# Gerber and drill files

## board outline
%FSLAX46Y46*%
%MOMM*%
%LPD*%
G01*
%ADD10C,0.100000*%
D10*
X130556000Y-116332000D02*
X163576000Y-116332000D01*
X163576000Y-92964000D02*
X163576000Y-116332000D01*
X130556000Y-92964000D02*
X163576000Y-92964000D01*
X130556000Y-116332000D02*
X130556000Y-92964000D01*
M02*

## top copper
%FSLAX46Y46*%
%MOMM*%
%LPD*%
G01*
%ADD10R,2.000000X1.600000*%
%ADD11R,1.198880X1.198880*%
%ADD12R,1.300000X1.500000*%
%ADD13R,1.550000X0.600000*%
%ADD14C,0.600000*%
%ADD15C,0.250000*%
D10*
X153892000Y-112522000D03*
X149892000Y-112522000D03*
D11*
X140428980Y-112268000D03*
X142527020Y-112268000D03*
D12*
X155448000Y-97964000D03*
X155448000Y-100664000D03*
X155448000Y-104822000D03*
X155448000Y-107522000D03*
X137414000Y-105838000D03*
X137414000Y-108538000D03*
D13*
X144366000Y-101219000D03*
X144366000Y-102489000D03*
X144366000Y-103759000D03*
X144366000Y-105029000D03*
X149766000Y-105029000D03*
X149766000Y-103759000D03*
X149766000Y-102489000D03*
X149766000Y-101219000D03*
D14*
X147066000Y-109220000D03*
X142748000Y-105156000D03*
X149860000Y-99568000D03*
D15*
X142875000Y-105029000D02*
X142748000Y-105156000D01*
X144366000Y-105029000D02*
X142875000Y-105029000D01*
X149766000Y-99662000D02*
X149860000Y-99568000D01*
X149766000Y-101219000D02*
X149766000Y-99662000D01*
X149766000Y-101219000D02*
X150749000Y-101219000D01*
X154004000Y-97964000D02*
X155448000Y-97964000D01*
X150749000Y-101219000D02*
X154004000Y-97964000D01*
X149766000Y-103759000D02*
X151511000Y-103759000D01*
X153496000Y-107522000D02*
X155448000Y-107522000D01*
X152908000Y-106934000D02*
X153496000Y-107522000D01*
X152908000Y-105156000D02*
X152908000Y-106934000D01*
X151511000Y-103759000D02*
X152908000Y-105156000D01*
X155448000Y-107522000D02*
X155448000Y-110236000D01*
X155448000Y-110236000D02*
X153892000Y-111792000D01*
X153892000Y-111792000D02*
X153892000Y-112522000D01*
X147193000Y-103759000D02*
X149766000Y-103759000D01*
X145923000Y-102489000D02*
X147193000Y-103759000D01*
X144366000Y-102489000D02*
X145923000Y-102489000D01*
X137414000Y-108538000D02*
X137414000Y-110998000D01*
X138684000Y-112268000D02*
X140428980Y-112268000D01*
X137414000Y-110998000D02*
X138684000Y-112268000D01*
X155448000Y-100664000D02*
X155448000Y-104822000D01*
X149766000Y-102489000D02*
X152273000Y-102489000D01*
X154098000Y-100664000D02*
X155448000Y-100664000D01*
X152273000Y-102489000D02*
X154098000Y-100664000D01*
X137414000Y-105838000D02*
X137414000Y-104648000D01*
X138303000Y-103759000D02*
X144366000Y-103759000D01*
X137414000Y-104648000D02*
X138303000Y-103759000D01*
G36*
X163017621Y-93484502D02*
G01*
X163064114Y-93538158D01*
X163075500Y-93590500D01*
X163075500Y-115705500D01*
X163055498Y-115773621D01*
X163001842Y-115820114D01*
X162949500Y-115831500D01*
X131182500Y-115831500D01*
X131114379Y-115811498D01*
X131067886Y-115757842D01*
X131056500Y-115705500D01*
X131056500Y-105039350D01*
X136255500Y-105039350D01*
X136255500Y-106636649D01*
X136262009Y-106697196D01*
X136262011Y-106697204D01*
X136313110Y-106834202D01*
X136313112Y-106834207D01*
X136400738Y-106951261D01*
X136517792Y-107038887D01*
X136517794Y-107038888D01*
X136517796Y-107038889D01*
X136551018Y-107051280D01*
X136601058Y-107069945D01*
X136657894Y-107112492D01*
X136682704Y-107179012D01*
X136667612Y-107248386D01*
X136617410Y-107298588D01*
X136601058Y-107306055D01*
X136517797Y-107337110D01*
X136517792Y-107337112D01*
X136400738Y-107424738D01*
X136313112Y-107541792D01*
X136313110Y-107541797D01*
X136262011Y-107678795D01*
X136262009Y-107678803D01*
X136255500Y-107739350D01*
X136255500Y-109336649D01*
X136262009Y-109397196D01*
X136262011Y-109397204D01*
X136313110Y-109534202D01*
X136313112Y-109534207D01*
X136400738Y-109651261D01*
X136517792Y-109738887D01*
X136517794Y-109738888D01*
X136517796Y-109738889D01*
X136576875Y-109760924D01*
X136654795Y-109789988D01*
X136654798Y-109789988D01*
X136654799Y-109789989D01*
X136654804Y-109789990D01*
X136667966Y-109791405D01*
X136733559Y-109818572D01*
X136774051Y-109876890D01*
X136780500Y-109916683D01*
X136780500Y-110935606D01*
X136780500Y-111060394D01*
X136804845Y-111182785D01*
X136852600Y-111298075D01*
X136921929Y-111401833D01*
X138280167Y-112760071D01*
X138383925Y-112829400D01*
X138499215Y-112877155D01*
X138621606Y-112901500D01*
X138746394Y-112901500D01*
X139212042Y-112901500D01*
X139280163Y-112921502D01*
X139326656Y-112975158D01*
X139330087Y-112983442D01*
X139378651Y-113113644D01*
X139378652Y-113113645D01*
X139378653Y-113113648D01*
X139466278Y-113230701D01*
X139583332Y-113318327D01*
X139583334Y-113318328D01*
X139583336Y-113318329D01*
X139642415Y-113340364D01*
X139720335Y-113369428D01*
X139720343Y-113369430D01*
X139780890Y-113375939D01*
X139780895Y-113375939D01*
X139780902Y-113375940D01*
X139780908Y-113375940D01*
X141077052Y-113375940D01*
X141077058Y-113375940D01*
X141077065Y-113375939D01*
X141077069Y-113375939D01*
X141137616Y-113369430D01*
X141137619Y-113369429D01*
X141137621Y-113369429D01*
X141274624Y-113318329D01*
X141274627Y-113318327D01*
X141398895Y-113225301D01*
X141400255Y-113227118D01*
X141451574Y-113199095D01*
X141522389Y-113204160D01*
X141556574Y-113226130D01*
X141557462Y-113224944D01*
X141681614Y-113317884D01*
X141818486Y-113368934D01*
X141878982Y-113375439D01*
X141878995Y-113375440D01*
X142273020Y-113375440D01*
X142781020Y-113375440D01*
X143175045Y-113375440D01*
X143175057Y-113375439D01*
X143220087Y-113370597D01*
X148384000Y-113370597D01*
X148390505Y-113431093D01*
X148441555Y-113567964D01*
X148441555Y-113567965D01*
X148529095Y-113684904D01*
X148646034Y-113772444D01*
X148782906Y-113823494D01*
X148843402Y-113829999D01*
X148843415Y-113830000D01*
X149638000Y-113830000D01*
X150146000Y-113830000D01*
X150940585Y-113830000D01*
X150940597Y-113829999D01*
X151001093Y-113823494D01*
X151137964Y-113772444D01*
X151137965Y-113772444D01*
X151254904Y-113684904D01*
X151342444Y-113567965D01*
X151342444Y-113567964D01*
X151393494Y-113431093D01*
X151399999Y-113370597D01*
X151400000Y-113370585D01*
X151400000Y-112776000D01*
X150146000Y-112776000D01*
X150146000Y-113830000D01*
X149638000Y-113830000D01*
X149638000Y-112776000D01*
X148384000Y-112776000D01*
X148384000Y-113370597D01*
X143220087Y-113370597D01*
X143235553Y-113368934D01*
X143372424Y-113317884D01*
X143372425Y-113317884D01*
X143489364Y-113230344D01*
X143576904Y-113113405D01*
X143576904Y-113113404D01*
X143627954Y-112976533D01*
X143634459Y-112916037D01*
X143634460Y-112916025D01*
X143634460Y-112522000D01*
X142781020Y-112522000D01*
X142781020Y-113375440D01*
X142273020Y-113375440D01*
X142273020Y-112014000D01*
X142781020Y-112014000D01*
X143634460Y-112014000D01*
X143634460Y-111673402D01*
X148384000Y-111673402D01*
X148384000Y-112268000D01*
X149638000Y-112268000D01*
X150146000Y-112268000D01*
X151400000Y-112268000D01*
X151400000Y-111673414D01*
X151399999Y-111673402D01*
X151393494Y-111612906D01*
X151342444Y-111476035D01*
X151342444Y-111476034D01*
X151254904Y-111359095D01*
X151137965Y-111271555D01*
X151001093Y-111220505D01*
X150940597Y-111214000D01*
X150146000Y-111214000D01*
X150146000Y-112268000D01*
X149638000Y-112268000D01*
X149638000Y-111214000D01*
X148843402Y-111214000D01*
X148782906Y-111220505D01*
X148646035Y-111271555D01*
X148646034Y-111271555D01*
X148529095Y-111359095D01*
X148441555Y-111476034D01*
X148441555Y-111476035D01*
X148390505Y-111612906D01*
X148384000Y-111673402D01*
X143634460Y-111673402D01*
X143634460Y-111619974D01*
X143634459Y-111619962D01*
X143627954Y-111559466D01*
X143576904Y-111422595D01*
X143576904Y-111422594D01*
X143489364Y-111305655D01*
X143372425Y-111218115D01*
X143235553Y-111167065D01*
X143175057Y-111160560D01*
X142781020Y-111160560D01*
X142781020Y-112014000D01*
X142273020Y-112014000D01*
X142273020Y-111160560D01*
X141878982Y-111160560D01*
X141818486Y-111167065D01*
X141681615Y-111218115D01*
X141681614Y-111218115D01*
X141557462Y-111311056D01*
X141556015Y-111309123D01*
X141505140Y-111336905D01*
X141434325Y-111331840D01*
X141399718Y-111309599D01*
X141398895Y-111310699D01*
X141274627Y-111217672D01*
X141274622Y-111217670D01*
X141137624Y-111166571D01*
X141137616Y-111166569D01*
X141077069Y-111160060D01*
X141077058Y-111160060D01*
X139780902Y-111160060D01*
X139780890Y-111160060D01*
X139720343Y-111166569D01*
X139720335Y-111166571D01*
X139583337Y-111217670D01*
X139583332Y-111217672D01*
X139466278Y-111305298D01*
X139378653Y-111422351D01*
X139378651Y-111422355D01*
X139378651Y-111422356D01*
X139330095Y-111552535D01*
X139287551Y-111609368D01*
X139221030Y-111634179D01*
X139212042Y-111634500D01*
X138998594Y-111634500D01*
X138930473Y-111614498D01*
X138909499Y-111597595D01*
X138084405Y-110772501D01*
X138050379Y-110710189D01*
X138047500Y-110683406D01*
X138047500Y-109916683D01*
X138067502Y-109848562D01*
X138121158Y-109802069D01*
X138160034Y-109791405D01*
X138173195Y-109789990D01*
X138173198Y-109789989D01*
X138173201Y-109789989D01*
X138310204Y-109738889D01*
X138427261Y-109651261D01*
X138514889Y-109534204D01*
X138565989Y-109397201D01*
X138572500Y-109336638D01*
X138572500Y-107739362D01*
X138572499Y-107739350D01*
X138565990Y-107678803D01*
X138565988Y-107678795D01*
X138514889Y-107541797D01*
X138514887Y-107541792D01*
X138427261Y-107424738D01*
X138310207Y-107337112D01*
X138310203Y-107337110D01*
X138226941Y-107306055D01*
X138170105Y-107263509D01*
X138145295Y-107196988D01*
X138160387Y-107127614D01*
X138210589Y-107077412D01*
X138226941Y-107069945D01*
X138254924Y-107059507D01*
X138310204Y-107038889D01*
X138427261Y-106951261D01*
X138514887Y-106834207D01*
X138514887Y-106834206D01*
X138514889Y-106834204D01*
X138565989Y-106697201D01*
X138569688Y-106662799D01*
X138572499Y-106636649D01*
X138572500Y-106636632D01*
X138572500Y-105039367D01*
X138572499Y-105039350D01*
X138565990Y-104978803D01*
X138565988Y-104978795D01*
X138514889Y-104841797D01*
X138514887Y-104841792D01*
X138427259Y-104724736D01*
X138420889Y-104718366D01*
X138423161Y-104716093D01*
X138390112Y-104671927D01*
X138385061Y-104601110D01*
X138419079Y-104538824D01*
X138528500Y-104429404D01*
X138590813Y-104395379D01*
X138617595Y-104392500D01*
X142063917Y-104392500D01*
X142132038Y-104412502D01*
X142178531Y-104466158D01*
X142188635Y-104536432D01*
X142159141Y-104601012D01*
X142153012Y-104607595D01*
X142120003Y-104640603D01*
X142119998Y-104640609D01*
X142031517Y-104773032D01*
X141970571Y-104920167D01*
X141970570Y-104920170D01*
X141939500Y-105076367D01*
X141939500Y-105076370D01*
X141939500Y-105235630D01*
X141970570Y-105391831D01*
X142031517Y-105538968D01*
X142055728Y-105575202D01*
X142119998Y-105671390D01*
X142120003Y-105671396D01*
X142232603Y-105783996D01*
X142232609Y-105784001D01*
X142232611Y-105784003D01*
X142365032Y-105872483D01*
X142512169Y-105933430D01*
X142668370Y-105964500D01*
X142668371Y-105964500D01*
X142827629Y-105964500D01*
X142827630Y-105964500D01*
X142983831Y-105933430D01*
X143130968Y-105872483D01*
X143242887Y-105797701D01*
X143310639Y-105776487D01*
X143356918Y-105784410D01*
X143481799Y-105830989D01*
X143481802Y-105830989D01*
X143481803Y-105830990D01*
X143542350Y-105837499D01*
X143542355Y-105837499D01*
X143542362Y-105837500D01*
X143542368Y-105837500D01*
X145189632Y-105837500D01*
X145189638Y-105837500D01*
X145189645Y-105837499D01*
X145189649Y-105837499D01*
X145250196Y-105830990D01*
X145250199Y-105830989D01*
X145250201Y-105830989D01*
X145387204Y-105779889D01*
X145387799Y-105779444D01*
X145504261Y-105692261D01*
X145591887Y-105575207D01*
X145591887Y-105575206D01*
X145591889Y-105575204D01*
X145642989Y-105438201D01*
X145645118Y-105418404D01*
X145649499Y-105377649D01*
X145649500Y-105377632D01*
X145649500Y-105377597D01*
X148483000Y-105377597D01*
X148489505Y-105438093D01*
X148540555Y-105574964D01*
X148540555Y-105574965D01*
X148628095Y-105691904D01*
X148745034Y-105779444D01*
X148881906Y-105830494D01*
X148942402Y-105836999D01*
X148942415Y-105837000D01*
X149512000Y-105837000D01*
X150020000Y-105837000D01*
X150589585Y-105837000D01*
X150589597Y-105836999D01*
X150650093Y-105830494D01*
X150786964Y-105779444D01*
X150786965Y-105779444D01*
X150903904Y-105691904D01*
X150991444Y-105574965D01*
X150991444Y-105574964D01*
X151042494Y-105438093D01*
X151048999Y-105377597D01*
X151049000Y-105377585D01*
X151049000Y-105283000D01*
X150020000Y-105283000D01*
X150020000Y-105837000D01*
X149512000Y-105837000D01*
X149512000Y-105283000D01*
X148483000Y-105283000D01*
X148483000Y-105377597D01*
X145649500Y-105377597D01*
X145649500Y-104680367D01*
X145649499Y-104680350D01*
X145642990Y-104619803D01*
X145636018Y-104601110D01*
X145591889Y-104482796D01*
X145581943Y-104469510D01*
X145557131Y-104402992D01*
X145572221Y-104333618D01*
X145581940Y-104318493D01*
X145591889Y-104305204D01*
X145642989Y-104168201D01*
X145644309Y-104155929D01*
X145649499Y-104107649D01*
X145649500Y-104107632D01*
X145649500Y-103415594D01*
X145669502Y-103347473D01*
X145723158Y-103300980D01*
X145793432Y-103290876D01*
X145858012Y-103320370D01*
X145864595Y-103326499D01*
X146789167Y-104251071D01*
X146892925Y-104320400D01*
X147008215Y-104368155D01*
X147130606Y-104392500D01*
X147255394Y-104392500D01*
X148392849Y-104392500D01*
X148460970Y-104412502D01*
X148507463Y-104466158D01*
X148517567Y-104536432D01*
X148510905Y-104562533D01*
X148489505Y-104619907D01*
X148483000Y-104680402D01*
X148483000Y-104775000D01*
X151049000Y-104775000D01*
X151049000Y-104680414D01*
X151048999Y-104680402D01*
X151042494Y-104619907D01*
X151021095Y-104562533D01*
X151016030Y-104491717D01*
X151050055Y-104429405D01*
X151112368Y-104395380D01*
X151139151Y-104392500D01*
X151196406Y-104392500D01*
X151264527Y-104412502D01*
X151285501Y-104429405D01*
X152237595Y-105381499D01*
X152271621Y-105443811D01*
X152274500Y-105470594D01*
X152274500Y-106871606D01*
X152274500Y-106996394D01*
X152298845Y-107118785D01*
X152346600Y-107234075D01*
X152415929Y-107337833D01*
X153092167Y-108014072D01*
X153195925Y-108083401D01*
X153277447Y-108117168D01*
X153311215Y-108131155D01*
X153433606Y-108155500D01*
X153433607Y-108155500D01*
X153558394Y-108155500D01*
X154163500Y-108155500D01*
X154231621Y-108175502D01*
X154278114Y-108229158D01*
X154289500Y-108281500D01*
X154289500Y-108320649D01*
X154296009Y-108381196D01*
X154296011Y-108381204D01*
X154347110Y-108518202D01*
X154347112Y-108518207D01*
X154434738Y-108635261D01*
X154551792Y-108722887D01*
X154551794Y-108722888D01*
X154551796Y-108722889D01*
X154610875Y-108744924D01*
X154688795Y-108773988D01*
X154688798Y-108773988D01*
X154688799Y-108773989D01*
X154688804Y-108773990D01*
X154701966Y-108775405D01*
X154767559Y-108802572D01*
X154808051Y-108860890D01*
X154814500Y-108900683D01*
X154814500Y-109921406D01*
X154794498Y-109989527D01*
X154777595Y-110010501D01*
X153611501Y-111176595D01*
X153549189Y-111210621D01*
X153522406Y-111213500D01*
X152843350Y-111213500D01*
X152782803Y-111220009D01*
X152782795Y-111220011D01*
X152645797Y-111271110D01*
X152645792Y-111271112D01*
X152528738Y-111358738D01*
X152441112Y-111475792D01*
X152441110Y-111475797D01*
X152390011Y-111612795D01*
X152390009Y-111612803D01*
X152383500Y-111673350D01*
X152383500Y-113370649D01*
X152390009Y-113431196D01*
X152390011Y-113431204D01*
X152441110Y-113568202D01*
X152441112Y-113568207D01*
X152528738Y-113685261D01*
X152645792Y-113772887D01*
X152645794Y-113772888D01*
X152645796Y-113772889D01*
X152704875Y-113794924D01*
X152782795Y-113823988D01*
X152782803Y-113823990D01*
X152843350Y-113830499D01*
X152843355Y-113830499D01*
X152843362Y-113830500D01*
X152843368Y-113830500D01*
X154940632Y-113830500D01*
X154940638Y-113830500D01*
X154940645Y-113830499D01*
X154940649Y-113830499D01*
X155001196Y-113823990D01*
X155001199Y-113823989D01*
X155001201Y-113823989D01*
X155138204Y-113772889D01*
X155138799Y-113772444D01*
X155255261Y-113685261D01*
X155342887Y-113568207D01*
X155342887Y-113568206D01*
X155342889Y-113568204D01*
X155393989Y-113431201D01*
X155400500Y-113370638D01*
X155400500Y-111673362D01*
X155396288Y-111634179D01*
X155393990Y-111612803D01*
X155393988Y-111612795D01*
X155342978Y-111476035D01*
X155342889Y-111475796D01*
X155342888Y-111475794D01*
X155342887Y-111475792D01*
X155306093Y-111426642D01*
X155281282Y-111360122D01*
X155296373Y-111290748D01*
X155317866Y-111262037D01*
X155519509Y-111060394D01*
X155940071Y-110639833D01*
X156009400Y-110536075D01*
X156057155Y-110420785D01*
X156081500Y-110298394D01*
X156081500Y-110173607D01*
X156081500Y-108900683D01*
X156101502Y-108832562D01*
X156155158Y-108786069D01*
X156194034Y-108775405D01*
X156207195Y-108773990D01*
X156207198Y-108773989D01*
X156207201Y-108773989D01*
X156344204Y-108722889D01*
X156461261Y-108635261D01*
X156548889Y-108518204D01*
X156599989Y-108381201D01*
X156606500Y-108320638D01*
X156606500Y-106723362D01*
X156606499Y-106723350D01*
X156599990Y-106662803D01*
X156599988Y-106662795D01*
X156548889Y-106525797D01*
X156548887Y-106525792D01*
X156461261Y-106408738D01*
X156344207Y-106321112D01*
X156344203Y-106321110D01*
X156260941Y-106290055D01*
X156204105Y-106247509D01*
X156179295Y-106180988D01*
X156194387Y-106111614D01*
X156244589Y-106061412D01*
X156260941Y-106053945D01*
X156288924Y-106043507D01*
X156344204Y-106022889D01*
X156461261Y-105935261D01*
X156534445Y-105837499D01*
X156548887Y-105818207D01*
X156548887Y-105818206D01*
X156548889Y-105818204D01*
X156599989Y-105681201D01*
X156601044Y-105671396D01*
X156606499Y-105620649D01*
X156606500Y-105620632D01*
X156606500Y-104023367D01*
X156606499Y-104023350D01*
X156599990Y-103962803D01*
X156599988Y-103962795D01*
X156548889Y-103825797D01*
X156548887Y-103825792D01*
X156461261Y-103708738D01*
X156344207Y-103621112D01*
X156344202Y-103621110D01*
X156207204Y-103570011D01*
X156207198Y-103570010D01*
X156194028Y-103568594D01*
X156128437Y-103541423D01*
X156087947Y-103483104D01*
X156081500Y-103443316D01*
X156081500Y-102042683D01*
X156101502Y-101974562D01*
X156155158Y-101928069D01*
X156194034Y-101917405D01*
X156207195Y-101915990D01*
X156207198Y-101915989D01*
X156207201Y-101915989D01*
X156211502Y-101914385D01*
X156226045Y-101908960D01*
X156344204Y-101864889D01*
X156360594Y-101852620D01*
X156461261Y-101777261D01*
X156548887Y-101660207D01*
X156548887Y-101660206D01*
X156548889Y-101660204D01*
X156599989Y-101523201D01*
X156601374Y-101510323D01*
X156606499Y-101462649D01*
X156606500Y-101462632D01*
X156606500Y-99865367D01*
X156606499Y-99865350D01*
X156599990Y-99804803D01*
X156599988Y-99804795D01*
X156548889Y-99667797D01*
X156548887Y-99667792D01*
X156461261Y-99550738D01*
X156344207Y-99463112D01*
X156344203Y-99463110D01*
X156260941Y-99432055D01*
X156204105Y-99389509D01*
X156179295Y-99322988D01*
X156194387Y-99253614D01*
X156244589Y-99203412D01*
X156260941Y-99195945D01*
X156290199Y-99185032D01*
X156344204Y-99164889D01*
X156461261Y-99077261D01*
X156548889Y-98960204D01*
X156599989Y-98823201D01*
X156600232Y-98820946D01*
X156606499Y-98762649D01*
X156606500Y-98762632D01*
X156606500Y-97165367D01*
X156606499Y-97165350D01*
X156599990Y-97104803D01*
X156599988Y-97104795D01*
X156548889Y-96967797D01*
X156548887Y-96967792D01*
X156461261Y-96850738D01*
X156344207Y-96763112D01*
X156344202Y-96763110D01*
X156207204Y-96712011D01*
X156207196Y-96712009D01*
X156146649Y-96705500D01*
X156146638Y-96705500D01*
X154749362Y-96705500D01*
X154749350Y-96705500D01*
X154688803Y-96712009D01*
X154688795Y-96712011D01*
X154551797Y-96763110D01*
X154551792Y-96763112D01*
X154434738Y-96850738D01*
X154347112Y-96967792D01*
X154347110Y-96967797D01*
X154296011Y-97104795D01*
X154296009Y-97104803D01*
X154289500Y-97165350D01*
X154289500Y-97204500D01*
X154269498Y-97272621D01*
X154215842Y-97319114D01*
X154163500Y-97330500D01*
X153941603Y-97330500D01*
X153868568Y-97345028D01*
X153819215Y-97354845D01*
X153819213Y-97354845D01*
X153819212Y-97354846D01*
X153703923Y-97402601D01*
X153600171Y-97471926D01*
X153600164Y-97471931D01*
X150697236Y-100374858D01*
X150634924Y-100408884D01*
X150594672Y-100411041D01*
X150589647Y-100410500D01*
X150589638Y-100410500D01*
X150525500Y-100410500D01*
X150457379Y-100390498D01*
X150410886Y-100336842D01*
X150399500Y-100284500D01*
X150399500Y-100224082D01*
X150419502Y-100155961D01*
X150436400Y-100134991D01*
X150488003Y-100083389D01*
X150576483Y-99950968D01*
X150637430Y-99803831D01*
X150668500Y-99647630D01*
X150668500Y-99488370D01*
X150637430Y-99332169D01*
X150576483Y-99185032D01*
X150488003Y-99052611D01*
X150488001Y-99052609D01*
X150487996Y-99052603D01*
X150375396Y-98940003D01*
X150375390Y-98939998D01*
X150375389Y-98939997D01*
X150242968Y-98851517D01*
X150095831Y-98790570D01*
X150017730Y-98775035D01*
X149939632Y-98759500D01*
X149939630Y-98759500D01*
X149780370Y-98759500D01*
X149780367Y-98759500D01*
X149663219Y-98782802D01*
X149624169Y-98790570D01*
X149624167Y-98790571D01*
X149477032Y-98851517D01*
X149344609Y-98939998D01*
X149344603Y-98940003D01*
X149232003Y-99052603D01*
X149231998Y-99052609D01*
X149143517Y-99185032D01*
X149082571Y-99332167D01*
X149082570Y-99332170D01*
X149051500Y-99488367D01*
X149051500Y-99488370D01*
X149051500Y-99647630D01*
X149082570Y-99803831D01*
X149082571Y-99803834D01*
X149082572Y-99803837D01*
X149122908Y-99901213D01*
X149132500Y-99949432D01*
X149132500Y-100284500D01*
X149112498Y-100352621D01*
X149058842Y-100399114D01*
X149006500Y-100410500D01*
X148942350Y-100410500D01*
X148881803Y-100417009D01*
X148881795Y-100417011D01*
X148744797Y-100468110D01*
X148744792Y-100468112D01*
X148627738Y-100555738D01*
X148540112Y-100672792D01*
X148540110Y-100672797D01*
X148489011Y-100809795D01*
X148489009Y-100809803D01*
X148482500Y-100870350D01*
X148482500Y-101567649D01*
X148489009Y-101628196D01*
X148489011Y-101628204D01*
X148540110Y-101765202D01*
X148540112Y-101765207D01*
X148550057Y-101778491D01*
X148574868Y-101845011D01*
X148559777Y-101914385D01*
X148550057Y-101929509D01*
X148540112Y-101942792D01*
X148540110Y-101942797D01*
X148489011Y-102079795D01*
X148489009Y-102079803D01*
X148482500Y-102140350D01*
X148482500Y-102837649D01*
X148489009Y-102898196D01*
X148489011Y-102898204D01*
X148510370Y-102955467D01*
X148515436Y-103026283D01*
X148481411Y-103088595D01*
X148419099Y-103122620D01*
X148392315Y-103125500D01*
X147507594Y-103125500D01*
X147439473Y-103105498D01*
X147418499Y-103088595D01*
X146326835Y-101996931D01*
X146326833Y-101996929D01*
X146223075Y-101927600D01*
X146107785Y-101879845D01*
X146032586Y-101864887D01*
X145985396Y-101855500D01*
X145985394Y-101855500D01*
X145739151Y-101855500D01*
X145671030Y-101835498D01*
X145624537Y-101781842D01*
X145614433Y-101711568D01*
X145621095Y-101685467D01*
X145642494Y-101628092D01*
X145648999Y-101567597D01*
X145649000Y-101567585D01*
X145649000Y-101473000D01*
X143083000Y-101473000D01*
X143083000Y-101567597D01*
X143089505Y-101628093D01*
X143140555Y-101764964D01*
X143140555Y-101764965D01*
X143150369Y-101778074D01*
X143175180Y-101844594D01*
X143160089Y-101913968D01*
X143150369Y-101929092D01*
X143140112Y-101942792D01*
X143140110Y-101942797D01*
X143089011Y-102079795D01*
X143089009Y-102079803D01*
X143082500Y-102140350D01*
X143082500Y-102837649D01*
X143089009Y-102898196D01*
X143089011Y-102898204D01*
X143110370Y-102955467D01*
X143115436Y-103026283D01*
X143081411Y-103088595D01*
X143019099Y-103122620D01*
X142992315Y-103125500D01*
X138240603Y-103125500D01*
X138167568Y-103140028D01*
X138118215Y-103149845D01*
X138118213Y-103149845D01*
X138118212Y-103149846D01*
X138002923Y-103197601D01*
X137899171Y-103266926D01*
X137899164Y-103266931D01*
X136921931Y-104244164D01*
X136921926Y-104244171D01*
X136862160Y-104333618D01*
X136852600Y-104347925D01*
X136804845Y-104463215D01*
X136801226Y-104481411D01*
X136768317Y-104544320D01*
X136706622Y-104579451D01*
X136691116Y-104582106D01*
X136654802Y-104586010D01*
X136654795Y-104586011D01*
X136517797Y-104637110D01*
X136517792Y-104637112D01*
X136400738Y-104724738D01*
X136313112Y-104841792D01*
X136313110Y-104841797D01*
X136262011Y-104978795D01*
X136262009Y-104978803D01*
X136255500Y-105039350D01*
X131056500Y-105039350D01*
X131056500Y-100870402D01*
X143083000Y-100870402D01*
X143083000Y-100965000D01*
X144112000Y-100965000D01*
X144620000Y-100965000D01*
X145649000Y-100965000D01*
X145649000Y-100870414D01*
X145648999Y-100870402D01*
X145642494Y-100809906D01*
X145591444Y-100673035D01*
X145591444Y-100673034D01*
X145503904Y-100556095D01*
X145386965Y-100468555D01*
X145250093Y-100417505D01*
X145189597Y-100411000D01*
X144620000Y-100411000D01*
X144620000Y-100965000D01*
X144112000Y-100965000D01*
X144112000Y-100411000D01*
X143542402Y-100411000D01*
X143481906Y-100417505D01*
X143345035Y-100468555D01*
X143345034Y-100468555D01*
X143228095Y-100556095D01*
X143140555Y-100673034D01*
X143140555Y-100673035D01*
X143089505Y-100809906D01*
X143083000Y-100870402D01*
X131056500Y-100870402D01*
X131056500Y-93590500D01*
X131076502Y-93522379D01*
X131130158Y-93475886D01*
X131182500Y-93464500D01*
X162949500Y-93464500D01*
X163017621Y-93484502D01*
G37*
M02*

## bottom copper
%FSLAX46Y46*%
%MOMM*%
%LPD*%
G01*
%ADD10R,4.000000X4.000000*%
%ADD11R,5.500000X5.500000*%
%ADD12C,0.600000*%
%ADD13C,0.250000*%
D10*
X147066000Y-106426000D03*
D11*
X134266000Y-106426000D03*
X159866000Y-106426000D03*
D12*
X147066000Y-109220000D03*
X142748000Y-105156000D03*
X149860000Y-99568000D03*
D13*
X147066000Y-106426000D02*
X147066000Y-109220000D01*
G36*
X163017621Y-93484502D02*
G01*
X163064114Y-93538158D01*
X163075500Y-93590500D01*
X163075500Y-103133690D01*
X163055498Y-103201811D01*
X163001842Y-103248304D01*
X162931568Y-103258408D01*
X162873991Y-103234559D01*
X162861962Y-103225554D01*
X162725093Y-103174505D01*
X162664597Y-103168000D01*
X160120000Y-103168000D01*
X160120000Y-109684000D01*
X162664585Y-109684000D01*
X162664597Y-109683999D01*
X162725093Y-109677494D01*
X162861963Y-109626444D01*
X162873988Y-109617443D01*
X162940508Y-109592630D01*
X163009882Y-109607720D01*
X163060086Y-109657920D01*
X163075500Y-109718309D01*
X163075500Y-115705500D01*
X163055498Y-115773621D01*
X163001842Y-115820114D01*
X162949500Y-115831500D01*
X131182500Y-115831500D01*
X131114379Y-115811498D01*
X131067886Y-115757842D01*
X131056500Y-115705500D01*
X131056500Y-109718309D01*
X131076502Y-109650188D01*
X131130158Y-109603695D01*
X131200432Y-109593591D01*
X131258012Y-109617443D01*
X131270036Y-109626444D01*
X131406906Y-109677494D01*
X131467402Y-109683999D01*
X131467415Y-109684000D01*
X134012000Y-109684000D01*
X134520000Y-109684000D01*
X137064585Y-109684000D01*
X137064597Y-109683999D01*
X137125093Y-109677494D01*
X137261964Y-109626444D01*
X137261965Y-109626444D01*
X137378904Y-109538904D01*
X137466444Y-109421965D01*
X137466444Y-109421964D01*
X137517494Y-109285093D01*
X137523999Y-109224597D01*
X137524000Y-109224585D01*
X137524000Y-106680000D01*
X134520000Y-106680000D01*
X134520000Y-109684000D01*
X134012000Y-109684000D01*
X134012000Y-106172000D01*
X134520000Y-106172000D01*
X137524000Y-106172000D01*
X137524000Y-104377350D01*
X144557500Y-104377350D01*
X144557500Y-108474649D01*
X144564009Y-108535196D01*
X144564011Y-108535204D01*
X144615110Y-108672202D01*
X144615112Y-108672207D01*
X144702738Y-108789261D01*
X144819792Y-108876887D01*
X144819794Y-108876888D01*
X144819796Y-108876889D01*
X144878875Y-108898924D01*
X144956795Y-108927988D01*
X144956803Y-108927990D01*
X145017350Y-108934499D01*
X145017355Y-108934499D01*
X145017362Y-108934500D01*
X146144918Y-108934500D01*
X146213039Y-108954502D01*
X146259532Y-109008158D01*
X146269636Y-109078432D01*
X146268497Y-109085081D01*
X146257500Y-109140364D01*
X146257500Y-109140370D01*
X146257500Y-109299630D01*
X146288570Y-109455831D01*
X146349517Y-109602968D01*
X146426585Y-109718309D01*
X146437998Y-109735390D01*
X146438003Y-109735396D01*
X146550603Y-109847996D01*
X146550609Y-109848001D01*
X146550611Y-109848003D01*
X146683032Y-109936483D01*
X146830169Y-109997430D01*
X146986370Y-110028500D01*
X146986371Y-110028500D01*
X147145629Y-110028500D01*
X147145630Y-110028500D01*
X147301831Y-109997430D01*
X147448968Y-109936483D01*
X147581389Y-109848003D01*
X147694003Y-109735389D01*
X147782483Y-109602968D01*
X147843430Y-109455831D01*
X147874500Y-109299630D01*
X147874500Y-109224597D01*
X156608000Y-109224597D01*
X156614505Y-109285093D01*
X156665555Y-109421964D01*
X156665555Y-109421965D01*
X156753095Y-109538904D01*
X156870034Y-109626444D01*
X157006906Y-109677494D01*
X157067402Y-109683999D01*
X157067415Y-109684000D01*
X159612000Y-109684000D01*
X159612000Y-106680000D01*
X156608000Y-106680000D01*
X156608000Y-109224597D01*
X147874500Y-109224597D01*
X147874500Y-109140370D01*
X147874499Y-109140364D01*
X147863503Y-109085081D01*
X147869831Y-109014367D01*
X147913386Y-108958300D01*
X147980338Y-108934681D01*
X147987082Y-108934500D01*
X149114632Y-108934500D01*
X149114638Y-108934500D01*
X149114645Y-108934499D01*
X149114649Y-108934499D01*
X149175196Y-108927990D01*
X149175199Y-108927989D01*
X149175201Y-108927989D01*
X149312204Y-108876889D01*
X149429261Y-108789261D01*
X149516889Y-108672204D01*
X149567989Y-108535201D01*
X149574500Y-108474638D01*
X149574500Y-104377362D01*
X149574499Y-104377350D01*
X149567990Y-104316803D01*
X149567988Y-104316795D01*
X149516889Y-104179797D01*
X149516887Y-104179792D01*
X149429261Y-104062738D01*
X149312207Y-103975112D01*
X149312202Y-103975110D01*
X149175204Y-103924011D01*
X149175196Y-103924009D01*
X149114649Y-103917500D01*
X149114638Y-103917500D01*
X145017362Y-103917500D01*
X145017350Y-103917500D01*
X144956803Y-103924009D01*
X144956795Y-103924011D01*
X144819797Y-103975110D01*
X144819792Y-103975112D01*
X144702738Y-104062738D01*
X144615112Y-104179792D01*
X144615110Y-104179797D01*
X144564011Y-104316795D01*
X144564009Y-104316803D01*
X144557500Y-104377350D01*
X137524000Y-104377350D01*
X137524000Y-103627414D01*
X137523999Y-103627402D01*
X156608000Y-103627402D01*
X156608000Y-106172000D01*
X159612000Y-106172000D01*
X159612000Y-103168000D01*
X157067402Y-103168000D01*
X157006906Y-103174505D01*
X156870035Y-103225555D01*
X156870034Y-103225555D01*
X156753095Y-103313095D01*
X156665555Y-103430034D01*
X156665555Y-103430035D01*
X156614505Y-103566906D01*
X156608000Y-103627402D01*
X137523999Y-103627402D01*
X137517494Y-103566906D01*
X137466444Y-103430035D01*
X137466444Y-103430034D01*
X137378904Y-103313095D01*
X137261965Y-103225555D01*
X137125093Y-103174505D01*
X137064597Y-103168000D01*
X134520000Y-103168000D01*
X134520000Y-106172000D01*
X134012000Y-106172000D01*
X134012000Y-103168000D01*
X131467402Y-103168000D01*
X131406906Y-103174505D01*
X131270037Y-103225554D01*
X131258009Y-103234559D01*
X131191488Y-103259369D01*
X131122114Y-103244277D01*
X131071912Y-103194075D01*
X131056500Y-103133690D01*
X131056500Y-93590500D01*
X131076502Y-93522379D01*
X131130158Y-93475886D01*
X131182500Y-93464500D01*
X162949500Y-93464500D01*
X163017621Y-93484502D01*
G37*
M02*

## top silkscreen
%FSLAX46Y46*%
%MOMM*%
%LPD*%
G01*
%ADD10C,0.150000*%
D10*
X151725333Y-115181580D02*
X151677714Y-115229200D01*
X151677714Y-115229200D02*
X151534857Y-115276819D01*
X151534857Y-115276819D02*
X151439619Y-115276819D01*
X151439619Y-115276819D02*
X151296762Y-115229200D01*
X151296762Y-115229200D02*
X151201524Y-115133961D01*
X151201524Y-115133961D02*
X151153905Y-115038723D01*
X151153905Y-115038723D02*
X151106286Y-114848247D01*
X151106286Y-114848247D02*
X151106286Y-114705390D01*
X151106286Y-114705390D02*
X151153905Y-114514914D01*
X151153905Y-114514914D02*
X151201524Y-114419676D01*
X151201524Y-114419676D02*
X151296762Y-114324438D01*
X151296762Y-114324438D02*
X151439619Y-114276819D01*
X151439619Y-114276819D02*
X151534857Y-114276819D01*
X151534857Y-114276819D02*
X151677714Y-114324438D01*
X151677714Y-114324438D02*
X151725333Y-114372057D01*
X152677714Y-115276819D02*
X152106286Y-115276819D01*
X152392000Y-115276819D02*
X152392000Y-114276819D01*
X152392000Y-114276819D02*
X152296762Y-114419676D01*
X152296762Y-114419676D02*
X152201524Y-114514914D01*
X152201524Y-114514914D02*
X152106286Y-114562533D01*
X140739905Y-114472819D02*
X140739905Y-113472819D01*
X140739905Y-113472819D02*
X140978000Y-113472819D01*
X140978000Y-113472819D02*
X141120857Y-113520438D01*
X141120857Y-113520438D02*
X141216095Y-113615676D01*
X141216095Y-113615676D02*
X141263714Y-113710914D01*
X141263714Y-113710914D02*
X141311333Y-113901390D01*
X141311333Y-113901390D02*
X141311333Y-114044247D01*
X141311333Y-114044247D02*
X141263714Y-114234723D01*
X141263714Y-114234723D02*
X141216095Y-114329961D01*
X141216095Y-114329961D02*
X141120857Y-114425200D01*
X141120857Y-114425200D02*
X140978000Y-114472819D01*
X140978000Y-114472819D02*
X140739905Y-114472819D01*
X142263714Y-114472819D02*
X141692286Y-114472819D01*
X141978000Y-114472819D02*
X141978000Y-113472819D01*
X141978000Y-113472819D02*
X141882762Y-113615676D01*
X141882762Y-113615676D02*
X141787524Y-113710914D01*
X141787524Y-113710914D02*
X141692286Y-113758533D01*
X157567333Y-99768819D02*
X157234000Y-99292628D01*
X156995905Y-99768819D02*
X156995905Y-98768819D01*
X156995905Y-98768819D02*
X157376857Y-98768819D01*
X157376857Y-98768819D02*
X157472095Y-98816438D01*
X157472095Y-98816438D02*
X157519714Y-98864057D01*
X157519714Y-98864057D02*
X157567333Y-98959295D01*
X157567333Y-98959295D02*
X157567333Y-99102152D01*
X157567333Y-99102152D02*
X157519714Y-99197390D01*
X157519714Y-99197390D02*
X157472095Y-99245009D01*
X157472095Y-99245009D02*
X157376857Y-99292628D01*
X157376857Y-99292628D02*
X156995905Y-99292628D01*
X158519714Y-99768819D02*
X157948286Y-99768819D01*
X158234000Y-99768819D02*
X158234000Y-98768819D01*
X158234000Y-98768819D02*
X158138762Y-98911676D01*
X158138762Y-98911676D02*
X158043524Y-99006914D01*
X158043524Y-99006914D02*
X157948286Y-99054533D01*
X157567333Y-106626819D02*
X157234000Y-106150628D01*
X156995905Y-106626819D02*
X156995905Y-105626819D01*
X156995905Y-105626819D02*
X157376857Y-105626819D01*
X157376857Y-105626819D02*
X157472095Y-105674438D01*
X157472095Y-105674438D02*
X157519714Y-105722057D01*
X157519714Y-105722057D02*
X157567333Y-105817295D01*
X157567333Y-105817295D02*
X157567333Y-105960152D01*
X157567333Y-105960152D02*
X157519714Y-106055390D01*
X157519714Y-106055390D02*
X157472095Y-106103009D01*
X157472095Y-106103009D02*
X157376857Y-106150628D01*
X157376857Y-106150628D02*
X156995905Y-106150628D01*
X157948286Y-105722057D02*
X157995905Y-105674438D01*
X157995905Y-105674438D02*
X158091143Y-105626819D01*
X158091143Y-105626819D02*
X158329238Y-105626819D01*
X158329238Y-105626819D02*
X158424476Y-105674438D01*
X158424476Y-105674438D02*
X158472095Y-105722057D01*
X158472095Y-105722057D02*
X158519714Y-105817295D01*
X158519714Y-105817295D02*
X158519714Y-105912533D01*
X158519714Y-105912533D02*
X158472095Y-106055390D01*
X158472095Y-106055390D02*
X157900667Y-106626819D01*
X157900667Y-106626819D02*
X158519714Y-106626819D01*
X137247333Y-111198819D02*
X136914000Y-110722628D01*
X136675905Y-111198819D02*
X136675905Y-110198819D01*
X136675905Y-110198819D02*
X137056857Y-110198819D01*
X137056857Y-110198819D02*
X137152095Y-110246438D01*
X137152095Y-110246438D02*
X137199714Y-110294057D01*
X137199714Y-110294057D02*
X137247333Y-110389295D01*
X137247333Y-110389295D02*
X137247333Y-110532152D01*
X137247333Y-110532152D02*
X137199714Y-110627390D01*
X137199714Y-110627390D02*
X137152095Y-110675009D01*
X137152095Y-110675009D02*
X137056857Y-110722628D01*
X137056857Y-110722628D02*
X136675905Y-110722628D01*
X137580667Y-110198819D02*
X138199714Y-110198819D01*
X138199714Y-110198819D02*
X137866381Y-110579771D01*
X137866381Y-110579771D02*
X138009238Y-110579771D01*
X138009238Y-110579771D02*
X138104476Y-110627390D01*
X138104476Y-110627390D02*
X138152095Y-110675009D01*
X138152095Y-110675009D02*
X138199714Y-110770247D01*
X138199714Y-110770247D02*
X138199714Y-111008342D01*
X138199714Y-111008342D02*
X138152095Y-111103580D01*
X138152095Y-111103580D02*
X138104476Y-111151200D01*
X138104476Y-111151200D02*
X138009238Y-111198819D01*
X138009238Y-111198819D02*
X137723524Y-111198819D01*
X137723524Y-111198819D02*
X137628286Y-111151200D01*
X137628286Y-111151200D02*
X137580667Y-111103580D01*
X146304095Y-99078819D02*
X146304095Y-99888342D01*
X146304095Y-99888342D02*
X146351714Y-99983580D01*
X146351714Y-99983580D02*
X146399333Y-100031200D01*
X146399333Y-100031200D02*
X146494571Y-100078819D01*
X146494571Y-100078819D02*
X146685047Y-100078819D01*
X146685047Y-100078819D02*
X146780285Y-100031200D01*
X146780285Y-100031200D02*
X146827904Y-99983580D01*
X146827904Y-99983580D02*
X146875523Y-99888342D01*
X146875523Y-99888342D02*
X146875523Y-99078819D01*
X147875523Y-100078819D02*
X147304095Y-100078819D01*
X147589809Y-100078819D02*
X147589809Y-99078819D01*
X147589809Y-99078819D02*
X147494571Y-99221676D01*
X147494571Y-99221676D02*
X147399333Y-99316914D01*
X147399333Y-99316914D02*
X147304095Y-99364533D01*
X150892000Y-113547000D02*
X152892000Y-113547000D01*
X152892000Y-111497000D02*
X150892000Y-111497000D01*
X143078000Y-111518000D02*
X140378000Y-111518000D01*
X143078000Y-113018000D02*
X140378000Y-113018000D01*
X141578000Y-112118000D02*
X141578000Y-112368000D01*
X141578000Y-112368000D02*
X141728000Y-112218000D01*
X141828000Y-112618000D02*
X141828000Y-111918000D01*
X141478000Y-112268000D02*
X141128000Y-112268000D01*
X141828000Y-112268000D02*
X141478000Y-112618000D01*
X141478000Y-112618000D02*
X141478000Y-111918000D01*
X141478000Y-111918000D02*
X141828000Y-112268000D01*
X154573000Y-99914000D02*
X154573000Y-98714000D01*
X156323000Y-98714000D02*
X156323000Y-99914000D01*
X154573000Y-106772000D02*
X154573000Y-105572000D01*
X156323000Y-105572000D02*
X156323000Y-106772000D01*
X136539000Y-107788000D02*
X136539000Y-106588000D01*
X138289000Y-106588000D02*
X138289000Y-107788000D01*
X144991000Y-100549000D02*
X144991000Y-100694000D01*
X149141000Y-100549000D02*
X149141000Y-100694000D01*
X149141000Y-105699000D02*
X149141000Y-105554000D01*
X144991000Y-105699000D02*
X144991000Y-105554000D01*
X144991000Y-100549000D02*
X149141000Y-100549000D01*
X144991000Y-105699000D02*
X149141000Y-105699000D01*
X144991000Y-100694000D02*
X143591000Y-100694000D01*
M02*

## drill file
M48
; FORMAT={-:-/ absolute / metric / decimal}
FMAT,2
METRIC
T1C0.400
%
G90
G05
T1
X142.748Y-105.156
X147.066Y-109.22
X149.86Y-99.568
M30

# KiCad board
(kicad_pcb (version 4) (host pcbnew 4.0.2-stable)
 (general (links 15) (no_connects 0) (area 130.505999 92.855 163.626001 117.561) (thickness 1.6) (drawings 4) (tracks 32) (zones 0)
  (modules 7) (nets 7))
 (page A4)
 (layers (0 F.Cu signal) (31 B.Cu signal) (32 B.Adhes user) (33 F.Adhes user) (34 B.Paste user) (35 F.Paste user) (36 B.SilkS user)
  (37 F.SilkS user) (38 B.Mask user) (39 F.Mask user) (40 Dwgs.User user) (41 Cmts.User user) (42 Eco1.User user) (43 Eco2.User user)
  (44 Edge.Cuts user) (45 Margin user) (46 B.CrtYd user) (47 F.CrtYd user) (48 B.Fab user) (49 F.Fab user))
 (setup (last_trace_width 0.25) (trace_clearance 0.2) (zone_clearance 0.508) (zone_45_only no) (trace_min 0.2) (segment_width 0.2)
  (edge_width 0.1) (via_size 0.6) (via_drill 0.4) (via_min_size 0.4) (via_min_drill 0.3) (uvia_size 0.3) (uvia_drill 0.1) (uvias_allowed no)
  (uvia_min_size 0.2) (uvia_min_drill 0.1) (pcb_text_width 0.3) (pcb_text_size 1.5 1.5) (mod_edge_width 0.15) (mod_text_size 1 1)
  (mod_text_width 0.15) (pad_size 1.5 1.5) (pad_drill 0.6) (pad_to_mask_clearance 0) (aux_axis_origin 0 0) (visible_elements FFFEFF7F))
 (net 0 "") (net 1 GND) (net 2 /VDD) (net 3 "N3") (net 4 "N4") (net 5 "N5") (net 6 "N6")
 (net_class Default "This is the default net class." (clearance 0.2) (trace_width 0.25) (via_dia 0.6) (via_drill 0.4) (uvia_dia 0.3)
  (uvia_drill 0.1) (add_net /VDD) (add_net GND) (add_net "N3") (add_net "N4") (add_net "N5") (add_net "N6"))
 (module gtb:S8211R (layer B.Cu) (at 147.066 106.426)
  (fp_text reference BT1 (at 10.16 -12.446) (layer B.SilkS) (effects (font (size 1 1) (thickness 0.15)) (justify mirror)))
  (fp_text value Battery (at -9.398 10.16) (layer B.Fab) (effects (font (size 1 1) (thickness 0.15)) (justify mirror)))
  (pad 2 smd rect (at 0 0) (size 4 4) (layers B.Cu B.Paste B.Mask) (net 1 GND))
  (pad 1 smd rect (at -12.8 0) (size 5.5 5.5) (layers B.Cu B.Paste B.Mask) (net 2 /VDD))
  (pad 1 smd rect (at 12.8 0) (size 5.5 5.5) (layers B.Cu B.Paste B.Mask) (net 2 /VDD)))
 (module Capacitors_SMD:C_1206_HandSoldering (layer F.Cu) (at 151.892 112.522 180)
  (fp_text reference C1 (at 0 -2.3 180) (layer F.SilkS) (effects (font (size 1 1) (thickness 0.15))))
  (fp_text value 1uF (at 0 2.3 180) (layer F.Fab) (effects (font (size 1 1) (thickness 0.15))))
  (fp_line (start 1 -1.025) (end -1 -1.025) (layer F.SilkS) (width 0.15))
  (fp_line (start -1 1.025) (end 1 1.025) (layer F.SilkS) (width 0.15))
  (pad 1 smd rect (at -2 0 180) (size 2 1.6) (layers F.Cu F.Paste F.Mask) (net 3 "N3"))
  (pad 2 smd rect (at 2 0 180) (size 2 1.6) (layers F.Cu F.Paste F.Mask) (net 1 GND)))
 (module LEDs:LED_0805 (layer F.Cu) (at 141.478 112.268 180)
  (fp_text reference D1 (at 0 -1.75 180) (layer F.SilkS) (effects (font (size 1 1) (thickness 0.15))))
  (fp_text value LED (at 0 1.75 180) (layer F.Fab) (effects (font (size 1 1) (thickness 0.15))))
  (fp_line (start -1.6 0.75) (end 1.1 0.75) (layer F.SilkS) (width 0.15))
  (fp_line (start -1.6 -0.75) (end 1.1 -0.75) (layer F.SilkS) (width 0.15))
  (fp_line (start -0.1 0.15) (end -0.1 -0.1) (layer F.SilkS) (width 0.15))
  (fp_line (start -0.1 -0.1) (end -0.25 0.05) (layer F.SilkS) (width 0.15))
  (fp_line (start -0.35 -0.35) (end -0.35 0.35) (layer F.SilkS) (width 0.15))
  (fp_line (start 0 0) (end 0.35 0) (layer F.SilkS) (width 0.15))
  (fp_line (start -0.35 0) (end 0 -0.35) (layer F.SilkS) (width 0.15))
  (fp_line (start 0 -0.35) (end 0 0.35) (layer F.SilkS) (width 0.15))
  (fp_line (start 0 0.35) (end -0.35 0) (layer F.SilkS) (width 0.15))
  (pad 2 smd rect (at 1.04902 0) (size 1.19888 1.19888) (layers F.Cu F.Paste F.Mask) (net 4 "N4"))
  (pad 1 smd rect (at -1.04902 0) (size 1.19888 1.19888) (layers F.Cu F.Paste F.Mask) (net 1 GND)))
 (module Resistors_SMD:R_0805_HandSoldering (layer F.Cu) (at 155.448 99.314 270)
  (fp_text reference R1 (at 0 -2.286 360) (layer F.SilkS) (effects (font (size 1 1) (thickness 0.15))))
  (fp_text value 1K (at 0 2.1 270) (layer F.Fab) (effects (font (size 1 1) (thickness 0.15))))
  (fp_line (start 0.6 0.875) (end -0.6 0.875) (layer F.SilkS) (width 0.15))
  (fp_line (start -0.6 -0.875) (end 0.6 -0.875) (layer F.SilkS) (width 0.15))
  (pad 1 smd rect (at -1.35 0 270) (size 1.5 1.3) (layers F.Cu F.Paste F.Mask) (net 2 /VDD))
  (pad 2 smd rect (at 1.35 0 270) (size 1.5 1.3) (layers F.Cu F.Paste F.Mask) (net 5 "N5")))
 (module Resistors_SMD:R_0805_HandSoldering (layer F.Cu) (at 155.448 106.172 270)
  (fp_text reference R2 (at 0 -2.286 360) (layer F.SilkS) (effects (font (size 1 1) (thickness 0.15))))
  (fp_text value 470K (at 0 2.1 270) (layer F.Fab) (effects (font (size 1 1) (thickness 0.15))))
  (fp_line (start 0.6 0.875) (end -0.6 0.875) (layer F.SilkS) (width 0.15))
  (fp_line (start -0.6 -0.875) (end 0.6 -0.875) (layer F.SilkS) (width 0.15))
  (pad 1 smd rect (at -1.35 0 270) (size 1.5 1.3) (layers F.Cu F.Paste F.Mask) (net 5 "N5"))
  (pad 2 smd rect (at 1.35 0 270) (size 1.5 1.3) (layers F.Cu F.Paste F.Mask) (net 3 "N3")))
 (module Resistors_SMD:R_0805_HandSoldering (layer F.Cu) (at 137.414 107.188 270)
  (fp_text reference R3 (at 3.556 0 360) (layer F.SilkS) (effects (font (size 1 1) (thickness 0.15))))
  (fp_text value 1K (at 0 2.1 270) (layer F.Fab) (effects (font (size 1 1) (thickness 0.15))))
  (fp_line (start 0.6 0.875) (end -0.6 0.875) (layer F.SilkS) (width 0.15))
  (fp_line (start -0.6 -0.875) (end 0.6 -0.875) (layer F.SilkS) (width 0.15))
  (pad 1 smd rect (at -1.35 0 270) (size 1.5 1.3) (layers F.Cu F.Paste F.Mask) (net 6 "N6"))
  (pad 2 smd rect (at 1.35 0 270) (size 1.5 1.3) (layers F.Cu F.Paste F.Mask) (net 4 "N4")))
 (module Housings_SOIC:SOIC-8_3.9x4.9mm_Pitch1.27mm (layer F.Cu) (at 147.066 103.124)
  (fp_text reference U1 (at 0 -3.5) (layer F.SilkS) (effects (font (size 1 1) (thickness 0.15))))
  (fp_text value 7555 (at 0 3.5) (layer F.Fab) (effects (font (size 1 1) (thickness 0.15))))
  (fp_line (start -2.075 -2.575) (end -2.075 -2.43) (layer F.SilkS) (width 0.15))
  (fp_line (start 2.075 -2.575) (end 2.075 -2.43) (layer F.SilkS) (width 0.15))
  (fp_line (start 2.075 2.575) (end 2.075 2.43) (layer F.SilkS) (width 0.15))
  (fp_line (start -2.075 2.575) (end -2.075 2.43) (layer F.SilkS) (width 0.15))
  (fp_line (start -2.075 -2.575) (end 2.075 -2.575) (layer F.SilkS) (width 0.15))
  (fp_line (start -2.075 2.575) (end 2.075 2.575) (layer F.SilkS) (width 0.15))
  (fp_line (start -2.075 -2.43) (end -3.475 -2.43) (layer F.SilkS) (width 0.15))
  (pad 1 smd rect (at -2.7 -1.905) (size 1.55 0.6) (layers F.Cu F.Paste F.Mask) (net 1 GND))
  (pad 2 smd rect (at -2.7 -0.635) (size 1.55 0.6) (layers F.Cu F.Paste F.Mask) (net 3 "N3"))
  (pad 3 smd rect (at -2.7 0.635) (size 1.55 0.6) (layers F.Cu F.Paste F.Mask) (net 6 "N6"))
  (pad 4 smd rect (at -2.7 1.905) (size 1.55 0.6) (layers F.Cu F.Paste F.Mask) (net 2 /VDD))
  (pad 5 smd rect (at 2.7 1.905) (size 1.55 0.6) (layers F.Cu F.Paste F.Mask) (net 1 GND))
  (pad 6 smd rect (at 2.7 0.635) (size 1.55 0.6) (layers F.Cu F.Paste F.Mask) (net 3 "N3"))
  (pad 7 smd rect (at 2.7 -0.635) (size 1.55 0.6) (layers F.Cu F.Paste F.Mask) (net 5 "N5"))
  (pad 8 smd rect (at 2.7 -1.905) (size 1.55 0.6) (layers F.Cu F.Paste F.Mask) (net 2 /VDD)))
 (gr_line (start 130.556 116.332) (end 163.576 116.332) (angle 90) (layer Edge.Cuts) (width 0.1))
 (gr_line (start 163.576 92.964) (end 163.576 116.332) (angle 90) (layer Edge.Cuts) (width 0.1))
 (gr_line (start 130.556 92.964) (end 163.576 92.964) (angle 90) (layer Edge.Cuts) (width 0.1))
 (gr_line (start 130.556 116.332) (end 130.556 92.964) (angle 90) (layer Edge.Cuts) (width 0.1))
 (segment (start 147.066 106.426) (end 147.066 109.22) (width 0.25) (layer B.Cu) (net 1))
 (via (at 147.066 109.22) (size 0.6) (drill 0.4) (layers F.Cu B.Cu) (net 1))
 (via (at 142.748 105.156) (size 0.6) (drill 0.4) (layers F.Cu B.Cu) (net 2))
 (segment (start 142.875 105.029) (end 142.748 105.156) (width 0.25) (layer F.Cu) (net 2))
 (segment (start 144.366 105.029) (end 142.875 105.029) (width 0.25) (layer F.Cu) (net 2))
 (via (at 149.86 99.568) (size 0.6) (drill 0.4) (layers F.Cu B.Cu) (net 2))
 (segment (start 149.766 99.662) (end 149.86 99.568) (width 0.25) (layer F.Cu) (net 2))
 (segment (start 149.766 101.219) (end 149.766 99.662) (width 0.25) (layer F.Cu) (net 2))
 (segment (start 149.766 101.219) (end 150.749 101.219) (width 0.25) (layer F.Cu) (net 2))
 (segment (start 154.004 97.964) (end 155.448 97.964) (width 0.25) (layer F.Cu) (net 2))
 (segment (start 150.749 101.219) (end 154.004 97.964) (width 0.25) (layer F.Cu) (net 2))
 (segment (start 149.766 103.759) (end 151.511 103.759) (width 0.25) (layer F.Cu) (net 3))
 (segment (start 153.496 107.522) (end 155.448 107.522) (width 0.25) (layer F.Cu) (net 3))
 (segment (start 152.908 106.934) (end 153.496 107.522) (width 0.25) (layer F.Cu) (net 3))
 (segment (start 152.908 105.156) (end 152.908 106.934) (width 0.25) (layer F.Cu) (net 3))
 (segment (start 151.511 103.759) (end 152.908 105.156) (width 0.25) (layer F.Cu) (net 3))
 (segment (start 155.448 107.522) (end 155.448 110.236) (width 0.25) (layer F.Cu) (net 3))
 (segment (start 155.448 110.236) (end 153.892 111.792) (width 0.25) (layer F.Cu) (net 3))
 (segment (start 153.892 111.792) (end 153.892 112.522) (width 0.25) (layer F.Cu) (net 3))
 (segment (start 147.193 103.759) (end 149.766 103.759) (width 0.25) (layer F.Cu) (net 3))
 (segment (start 145.923 102.489) (end 147.193 103.759) (width 0.25) (layer F.Cu) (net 3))
 (segment (start 144.366 102.489) (end 145.923 102.489) (width 0.25) (layer F.Cu) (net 3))
 (segment (start 137.414 108.538) (end 137.414 110.998) (width 0.25) (layer F.Cu) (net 4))
 (segment (start 138.684 112.268) (end 140.42898 112.268) (width 0.25) (layer F.Cu) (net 4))
 (segment (start 137.414 110.998) (end 138.684 112.268) (width 0.25) (layer F.Cu) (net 4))
 (segment (start 155.448 100.664) (end 155.448 104.822) (width 0.25) (layer F.Cu) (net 5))
 (segment (start 149.766 102.489) (end 152.273 102.489) (width 0.25) (layer F.Cu) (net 5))
 (segment (start 154.098 100.664) (end 155.448 100.664) (width 0.25) (layer F.Cu) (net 5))
 (segment (start 152.273 102.489) (end 154.098 100.664) (width 0.25) (layer F.Cu) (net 5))
 (segment (start 137.414 105.838) (end 137.414 104.648) (width 0.25) (layer F.Cu) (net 6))
 (segment (start 138.303 103.759) (end 144.366 103.759) (width 0.25) (layer F.Cu) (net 6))
 (segment (start 137.414 104.648) (end 138.303 103.759) (width 0.25) (layer F.Cu) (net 6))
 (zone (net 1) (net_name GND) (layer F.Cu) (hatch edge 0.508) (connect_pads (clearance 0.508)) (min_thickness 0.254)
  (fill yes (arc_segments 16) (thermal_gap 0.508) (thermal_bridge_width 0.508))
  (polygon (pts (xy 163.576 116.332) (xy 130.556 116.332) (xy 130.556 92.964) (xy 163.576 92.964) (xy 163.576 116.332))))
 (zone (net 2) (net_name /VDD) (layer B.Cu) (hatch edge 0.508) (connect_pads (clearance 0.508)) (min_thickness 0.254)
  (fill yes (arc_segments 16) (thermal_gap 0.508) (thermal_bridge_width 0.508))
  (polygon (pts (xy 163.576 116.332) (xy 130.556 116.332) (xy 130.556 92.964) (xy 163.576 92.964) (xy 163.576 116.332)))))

